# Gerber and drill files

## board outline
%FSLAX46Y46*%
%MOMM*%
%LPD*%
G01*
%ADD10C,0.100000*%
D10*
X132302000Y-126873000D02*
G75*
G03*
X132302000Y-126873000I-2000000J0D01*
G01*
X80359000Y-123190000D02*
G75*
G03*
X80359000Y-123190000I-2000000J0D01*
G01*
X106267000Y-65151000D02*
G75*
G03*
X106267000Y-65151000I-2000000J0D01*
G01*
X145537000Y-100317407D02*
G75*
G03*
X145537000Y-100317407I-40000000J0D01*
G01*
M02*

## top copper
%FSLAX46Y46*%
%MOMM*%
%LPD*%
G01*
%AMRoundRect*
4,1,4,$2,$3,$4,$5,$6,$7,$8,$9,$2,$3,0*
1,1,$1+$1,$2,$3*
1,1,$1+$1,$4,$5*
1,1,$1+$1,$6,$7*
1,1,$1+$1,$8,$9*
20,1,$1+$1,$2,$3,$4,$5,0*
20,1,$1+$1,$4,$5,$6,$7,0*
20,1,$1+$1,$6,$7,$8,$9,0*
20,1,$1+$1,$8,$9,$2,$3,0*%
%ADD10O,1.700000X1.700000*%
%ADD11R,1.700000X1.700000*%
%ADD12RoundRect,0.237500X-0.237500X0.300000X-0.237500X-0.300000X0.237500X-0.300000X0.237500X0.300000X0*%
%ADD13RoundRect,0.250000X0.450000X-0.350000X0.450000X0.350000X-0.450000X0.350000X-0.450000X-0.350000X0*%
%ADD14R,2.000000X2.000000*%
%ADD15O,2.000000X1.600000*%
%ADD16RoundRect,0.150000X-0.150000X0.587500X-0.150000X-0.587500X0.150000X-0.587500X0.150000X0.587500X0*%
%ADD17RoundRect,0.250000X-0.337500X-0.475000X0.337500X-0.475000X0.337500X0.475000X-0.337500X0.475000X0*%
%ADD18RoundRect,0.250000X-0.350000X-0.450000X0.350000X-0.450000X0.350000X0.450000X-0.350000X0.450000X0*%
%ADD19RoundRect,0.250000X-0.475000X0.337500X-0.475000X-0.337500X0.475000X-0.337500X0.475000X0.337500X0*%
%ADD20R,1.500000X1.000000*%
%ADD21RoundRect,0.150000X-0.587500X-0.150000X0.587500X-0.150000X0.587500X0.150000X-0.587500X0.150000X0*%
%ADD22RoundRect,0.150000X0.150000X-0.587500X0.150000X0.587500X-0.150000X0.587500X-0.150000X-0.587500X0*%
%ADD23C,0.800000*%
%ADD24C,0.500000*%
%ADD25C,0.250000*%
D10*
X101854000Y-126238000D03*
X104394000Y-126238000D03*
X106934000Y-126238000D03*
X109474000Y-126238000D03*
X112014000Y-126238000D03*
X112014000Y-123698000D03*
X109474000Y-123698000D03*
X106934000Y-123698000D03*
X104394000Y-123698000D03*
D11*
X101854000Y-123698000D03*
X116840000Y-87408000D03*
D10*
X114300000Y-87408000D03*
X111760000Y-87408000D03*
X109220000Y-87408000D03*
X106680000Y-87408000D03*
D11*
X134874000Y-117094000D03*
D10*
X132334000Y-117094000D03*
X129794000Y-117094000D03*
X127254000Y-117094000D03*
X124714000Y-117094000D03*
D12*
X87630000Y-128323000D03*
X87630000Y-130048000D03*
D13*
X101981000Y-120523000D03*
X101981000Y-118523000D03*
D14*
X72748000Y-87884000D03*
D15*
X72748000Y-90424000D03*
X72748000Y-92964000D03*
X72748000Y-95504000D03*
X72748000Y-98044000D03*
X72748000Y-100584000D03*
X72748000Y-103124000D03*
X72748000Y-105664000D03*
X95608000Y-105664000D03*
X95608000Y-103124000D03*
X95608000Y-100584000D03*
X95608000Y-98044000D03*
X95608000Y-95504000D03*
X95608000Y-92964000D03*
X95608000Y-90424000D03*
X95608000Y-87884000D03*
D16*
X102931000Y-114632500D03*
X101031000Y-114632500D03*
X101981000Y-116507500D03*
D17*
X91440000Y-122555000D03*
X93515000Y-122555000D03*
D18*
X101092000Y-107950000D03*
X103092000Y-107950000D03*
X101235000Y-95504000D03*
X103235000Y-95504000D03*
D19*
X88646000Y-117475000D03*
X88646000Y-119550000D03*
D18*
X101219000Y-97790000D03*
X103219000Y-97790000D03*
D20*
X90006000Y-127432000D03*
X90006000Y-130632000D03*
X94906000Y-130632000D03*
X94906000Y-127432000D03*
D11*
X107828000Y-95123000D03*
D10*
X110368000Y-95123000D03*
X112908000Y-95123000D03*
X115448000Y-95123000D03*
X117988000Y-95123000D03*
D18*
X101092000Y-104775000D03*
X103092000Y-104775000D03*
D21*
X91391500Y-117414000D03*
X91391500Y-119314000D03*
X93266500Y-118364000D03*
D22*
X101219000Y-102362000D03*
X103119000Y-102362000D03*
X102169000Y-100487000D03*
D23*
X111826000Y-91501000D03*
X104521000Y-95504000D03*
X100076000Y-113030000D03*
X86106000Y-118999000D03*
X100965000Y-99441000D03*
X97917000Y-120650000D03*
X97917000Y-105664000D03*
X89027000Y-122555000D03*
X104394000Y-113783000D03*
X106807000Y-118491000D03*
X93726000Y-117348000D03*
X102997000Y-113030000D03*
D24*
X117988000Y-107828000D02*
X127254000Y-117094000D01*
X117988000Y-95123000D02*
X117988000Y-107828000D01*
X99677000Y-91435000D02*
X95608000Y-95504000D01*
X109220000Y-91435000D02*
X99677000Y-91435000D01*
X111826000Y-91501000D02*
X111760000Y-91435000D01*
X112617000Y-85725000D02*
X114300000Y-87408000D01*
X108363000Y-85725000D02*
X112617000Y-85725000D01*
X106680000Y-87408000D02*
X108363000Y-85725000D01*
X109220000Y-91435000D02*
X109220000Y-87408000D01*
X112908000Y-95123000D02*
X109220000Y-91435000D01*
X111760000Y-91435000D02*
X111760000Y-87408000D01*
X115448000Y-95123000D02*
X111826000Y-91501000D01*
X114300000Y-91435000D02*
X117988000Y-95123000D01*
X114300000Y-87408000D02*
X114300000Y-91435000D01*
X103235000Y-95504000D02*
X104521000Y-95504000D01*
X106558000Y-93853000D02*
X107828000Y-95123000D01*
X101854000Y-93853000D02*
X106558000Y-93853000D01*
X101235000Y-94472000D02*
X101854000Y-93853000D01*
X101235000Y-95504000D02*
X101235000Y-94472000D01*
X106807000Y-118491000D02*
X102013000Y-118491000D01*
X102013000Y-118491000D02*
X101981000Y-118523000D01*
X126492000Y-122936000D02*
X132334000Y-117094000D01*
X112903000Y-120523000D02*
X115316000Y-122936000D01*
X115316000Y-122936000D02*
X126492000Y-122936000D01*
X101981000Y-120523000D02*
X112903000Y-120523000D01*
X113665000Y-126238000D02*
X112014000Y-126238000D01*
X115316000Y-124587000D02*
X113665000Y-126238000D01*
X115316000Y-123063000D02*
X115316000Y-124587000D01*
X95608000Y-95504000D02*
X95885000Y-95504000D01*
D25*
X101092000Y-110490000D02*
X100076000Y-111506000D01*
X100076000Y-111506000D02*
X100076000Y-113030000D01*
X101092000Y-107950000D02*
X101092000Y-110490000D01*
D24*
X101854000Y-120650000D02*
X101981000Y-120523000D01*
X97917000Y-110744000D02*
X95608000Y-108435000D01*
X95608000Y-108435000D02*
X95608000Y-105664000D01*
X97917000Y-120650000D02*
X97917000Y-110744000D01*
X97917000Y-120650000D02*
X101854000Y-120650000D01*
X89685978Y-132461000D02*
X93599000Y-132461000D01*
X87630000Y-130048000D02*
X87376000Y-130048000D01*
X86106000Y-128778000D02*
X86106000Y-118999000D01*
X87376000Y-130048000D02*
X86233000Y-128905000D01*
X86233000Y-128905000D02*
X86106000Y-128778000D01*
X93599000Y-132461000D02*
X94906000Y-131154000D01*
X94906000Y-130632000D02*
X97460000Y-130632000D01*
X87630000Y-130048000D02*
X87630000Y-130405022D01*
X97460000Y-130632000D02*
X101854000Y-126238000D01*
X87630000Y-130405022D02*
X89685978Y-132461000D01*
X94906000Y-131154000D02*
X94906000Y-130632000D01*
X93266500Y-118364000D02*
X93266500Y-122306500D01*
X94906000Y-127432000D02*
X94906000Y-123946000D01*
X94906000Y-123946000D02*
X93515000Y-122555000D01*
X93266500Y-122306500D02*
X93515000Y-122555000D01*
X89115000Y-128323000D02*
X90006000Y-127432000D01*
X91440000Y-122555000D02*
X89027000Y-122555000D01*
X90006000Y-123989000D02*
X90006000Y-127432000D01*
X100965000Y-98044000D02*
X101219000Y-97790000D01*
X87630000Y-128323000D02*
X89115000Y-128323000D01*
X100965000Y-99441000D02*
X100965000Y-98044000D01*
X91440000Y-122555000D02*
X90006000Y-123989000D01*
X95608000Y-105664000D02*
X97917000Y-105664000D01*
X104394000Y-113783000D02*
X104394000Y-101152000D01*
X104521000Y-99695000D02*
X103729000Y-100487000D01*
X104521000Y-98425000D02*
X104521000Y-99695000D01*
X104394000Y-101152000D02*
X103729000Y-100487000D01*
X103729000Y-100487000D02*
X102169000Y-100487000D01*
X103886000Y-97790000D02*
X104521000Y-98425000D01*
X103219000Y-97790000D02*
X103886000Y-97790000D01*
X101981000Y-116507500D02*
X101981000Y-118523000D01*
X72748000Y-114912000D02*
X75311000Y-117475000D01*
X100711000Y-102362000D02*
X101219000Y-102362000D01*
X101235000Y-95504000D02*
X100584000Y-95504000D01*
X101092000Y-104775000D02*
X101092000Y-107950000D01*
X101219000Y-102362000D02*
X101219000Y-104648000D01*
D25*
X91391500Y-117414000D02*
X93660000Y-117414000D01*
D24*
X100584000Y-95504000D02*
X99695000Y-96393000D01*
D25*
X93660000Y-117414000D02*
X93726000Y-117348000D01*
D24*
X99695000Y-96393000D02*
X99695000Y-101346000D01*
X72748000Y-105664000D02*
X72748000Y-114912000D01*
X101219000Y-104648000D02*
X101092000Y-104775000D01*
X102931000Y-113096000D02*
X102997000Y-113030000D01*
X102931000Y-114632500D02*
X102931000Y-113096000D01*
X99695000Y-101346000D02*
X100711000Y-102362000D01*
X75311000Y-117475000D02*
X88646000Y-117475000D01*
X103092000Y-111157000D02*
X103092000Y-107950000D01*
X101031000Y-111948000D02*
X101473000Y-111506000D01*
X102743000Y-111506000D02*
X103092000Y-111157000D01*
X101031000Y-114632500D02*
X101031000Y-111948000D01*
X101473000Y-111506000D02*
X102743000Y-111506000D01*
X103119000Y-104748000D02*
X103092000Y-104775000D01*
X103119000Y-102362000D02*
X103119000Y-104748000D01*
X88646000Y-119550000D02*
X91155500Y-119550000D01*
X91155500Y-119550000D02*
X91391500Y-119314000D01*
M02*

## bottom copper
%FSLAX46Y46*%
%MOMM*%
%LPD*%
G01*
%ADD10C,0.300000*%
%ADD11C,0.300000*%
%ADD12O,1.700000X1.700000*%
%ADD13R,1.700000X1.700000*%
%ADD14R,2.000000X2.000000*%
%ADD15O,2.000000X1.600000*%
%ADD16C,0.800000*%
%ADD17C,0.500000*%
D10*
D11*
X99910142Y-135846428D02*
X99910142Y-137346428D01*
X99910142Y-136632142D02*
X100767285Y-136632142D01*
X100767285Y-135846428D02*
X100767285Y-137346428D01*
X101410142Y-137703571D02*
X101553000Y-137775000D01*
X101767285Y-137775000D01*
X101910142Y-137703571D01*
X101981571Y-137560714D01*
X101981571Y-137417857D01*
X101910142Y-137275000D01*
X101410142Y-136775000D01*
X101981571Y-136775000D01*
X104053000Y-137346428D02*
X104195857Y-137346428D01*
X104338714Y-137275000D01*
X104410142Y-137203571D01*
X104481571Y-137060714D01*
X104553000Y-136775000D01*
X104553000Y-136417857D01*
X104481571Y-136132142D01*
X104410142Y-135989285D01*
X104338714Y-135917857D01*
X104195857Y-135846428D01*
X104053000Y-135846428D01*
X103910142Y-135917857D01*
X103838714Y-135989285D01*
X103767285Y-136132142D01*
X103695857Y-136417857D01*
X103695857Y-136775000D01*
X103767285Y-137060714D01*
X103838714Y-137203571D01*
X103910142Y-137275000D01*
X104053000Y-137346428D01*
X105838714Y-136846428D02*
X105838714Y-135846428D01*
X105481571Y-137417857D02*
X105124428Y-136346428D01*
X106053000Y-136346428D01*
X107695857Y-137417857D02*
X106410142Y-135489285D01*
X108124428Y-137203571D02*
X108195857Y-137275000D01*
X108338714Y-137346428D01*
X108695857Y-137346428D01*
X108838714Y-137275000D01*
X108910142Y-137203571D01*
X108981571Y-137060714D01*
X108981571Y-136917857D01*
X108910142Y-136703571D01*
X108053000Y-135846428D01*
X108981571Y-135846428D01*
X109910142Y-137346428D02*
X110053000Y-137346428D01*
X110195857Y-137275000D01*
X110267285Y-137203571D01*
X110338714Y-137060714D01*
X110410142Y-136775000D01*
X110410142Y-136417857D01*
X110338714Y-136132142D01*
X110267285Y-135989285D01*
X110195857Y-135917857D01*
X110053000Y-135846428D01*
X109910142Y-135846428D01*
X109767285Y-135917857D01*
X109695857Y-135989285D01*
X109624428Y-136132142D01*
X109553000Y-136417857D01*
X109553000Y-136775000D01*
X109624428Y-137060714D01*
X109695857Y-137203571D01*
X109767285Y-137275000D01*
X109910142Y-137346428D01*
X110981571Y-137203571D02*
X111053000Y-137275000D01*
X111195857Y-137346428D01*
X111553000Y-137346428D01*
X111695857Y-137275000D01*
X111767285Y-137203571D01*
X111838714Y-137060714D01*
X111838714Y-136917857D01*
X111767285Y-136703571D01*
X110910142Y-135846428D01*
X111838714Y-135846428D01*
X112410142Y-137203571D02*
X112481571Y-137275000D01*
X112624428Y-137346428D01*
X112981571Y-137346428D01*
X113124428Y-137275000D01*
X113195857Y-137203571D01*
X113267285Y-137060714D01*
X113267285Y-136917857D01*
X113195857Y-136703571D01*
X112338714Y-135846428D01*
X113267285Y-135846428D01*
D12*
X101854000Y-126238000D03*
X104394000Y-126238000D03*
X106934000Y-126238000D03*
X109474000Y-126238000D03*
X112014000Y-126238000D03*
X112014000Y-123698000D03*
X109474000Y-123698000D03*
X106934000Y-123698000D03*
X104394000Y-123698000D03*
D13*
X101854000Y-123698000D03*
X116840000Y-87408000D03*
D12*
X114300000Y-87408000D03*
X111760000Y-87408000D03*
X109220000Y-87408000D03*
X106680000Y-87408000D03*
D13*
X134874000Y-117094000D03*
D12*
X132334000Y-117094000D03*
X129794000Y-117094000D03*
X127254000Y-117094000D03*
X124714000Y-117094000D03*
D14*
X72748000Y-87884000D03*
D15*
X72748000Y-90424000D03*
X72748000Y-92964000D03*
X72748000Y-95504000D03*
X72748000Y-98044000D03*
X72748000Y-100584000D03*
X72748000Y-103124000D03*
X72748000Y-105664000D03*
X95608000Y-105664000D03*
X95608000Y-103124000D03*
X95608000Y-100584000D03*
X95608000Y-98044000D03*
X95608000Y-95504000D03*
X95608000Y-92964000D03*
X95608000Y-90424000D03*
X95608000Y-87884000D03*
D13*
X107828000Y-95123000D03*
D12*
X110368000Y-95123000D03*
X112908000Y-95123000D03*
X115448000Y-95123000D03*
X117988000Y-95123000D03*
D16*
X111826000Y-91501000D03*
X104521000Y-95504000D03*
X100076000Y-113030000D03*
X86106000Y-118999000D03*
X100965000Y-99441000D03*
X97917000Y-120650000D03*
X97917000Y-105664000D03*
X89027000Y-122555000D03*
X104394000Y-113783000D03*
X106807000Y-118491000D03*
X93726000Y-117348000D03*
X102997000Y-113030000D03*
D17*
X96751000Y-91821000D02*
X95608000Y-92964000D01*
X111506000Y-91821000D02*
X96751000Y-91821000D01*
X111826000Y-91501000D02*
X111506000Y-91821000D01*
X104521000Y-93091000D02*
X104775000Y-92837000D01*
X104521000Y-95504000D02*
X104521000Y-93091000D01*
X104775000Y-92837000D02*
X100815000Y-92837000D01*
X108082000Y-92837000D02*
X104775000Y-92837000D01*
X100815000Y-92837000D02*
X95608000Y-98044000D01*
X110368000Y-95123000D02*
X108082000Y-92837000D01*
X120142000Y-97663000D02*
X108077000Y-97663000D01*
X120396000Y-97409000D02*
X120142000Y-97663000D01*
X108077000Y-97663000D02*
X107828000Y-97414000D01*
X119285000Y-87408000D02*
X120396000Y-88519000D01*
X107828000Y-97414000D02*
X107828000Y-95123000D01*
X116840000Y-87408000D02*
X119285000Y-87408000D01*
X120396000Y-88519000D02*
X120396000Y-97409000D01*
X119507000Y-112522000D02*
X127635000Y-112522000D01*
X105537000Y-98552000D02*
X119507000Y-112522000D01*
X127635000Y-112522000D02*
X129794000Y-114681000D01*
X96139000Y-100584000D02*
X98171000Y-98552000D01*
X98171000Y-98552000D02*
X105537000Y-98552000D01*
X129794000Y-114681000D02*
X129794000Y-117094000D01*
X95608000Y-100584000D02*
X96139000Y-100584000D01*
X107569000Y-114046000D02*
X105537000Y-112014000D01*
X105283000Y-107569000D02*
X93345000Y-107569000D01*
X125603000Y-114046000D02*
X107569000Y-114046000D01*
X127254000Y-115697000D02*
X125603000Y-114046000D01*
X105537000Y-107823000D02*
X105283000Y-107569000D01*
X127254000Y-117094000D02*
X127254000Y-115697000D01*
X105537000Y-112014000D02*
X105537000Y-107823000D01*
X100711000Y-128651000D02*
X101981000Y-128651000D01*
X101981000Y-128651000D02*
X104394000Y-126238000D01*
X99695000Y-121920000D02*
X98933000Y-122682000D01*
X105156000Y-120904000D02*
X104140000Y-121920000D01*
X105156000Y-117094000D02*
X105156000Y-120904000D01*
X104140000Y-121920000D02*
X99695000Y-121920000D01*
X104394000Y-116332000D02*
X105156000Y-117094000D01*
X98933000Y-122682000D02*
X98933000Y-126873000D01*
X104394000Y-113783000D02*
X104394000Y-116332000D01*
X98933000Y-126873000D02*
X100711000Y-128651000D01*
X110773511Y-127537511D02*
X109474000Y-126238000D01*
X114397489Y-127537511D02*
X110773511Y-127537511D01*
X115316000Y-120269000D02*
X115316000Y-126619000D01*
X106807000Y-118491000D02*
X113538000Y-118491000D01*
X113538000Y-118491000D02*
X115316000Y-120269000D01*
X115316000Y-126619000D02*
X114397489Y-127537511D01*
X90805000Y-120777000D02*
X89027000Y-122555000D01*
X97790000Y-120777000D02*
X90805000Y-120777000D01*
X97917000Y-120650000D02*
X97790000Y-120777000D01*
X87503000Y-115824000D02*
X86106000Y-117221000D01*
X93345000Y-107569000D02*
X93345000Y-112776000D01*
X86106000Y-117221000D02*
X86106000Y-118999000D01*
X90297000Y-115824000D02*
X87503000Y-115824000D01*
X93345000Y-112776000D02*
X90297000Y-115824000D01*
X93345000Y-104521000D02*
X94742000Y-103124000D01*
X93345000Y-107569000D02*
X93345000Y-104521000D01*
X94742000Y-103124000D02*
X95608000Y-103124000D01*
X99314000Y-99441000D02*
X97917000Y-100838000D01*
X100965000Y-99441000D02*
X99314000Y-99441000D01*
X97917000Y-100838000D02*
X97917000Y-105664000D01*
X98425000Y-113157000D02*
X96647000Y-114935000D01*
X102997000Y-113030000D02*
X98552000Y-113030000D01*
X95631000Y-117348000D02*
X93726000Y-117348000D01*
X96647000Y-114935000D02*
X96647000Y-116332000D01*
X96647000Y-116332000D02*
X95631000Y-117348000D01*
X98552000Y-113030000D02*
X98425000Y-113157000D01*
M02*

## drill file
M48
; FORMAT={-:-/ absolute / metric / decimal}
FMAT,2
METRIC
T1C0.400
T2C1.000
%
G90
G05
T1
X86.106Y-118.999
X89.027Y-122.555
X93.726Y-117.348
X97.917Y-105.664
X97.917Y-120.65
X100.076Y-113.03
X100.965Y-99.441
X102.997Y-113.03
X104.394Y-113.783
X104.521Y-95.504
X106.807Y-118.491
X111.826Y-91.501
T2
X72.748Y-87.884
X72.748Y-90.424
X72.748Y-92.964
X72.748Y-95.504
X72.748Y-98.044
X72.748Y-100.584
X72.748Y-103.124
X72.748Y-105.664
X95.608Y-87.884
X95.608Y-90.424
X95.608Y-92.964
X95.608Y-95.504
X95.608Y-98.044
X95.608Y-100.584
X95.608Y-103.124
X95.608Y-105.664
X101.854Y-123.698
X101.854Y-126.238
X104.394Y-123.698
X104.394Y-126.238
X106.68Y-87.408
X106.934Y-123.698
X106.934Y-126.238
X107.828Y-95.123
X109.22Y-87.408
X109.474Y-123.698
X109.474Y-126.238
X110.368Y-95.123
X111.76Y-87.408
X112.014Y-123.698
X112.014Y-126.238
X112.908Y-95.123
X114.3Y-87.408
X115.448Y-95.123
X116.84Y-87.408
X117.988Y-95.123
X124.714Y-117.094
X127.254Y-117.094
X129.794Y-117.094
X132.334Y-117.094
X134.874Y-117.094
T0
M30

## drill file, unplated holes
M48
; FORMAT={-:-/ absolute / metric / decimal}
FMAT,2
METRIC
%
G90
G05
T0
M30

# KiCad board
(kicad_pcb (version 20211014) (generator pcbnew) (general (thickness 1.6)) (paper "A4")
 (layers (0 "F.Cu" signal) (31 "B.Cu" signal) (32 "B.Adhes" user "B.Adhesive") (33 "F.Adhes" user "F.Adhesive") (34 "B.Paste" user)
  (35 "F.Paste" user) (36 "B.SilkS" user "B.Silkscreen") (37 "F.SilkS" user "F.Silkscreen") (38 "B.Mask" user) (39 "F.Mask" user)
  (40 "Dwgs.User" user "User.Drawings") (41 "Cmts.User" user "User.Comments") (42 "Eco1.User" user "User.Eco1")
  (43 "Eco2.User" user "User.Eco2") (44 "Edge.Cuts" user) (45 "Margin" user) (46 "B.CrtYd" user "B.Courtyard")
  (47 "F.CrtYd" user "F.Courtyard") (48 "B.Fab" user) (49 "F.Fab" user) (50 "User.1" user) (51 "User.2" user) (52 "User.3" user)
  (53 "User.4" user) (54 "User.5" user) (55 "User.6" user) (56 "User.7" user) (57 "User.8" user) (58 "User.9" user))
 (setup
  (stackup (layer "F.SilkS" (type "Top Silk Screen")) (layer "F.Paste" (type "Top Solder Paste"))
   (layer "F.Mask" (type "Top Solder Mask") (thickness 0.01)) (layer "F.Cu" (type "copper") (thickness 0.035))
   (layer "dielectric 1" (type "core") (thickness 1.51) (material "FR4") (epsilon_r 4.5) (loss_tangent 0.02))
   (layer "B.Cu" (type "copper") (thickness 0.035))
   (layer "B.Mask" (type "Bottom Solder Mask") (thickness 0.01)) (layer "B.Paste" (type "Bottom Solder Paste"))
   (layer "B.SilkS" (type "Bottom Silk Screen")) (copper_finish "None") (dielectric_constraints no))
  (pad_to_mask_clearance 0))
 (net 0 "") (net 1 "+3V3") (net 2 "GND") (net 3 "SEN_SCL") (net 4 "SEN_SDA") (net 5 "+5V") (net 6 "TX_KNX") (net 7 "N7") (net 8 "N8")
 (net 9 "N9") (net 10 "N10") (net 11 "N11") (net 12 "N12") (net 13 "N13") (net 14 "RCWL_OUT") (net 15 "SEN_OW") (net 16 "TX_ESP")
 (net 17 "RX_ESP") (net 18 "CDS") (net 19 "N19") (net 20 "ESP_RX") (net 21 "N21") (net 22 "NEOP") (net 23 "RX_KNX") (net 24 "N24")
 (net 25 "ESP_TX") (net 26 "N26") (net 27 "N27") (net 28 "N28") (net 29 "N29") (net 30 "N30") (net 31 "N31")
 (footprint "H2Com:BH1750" (layer "F.Cu") (at 116.84 100.108 -90)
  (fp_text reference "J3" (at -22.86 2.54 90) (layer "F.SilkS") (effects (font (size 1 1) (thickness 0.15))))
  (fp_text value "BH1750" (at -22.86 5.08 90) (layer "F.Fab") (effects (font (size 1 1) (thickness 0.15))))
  (pad "1" thru_hole rect (at -12.7 0 270) (size 1.7 1.7) (drill 1) (layers *.Cu *.Mask) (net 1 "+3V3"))
  (pad "2" thru_hole oval (at -12.7 2.54 270) (size 1.7 1.7) (drill 1) (layers *.Cu *.Mask) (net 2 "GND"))
  (pad "3" thru_hole oval (at -12.7 5.08 270) (size 1.7 1.7) (drill 1) (layers *.Cu *.Mask) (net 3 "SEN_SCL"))
  (pad "4" thru_hole oval (at -12.7 7.62 270) (size 1.7 1.7) (drill 1) (layers *.Cu *.Mask) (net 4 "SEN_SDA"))
  (pad "5" thru_hole oval (at -12.7 10.16 270) (size 1.7 1.7) (drill 1) (layers *.Cu *.Mask) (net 2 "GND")))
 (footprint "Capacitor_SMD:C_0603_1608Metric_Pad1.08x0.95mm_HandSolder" (layer "F.Cu") (at 87.63 129.1855 -90)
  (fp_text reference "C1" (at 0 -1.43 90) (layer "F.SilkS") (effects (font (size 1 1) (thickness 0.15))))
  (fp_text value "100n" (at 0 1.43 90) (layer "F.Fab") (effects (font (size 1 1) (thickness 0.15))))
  (pad "1" smd roundrect locked (at -0.8625 0 270) (size 1.075 0.95) (layers "F.Cu" "F.Paste" "F.Mask") (roundrect_rratio 0.25)
   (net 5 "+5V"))
  (pad "2" smd roundrect locked (at 0.8625 0 270) (size 1.075 0.95) (layers "F.Cu" "F.Paste" "F.Mask") (roundrect_rratio 0.25) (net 2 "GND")))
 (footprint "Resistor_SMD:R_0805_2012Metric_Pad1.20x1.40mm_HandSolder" (layer "F.Cu") (at 101.981 119.523 90)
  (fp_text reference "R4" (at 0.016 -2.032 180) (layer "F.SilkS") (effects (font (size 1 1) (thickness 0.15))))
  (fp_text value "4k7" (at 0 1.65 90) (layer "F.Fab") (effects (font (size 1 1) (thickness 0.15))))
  (pad "1" smd roundrect locked (at -1 0 90) (size 1.2 1.4) (layers "F.Cu" "F.Paste" "F.Mask") (roundrect_rratio 0.2083333333) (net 5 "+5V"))
  (pad "2" smd roundrect locked (at 1 0 90) (size 1.2 1.4) (layers "F.Cu" "F.Paste" "F.Mask") (roundrect_rratio 0.2083333333)
   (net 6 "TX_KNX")))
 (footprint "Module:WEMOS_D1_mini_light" (layer "F.Cu") (at 72.748 87.884)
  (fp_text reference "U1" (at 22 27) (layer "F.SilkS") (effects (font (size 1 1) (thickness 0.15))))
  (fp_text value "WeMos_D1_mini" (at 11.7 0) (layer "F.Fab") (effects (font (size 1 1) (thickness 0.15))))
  (pad "1" thru_hole rect locked (at 0 0) (size 2 2) (drill 1) (layers *.Cu *.Mask) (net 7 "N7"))
  (pad "2" thru_hole oval locked (at 0 2.54) (size 2 1.6) (drill 1) (layers *.Cu *.Mask) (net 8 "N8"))
  (pad "3" thru_hole oval locked (at 0 5.08) (size 2 1.6) (drill 1) (layers *.Cu *.Mask) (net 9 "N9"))
  (pad "4" thru_hole oval locked (at 0 7.62) (size 2 1.6) (drill 1) (layers *.Cu *.Mask) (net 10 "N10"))
  (pad "5" thru_hole oval locked (at 0 10.16) (size 2 1.6) (drill 1) (layers *.Cu *.Mask) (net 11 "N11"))
  (pad "6" thru_hole oval locked (at 0 12.7) (size 2 1.6) (drill 1) (layers *.Cu *.Mask) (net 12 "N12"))
  (pad "7" thru_hole oval locked (at 0 15.24) (size 2 1.6) (drill 1) (layers *.Cu *.Mask) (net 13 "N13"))
  (pad "8" thru_hole oval locked (at 0 17.78) (size 2 1.6) (drill 1) (layers *.Cu *.Mask) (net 1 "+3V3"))
  (pad "9" thru_hole oval locked (at 22.86 17.78) (size 2 1.6) (drill 1) (layers *.Cu *.Mask) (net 5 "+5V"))
  (pad "10" thru_hole oval locked (at 22.86 15.24) (size 2 1.6) (drill 1) (layers *.Cu *.Mask) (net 2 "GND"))
  (pad "11" thru_hole oval locked (at 22.86 12.7) (size 2 1.6) (drill 1) (layers *.Cu *.Mask) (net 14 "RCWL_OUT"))
  (pad "12" thru_hole oval locked (at 22.86 10.16) (size 2 1.6) (drill 1) (layers *.Cu *.Mask) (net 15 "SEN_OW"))
  (pad "13" thru_hole oval locked (at 22.86 7.62) (size 2 1.6) (drill 1) (layers *.Cu *.Mask) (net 4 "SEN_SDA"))
  (pad "14" thru_hole oval locked (at 22.86 5.08) (size 2 1.6) (drill 1) (layers *.Cu *.Mask) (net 3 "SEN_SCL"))
  (pad "15" thru_hole oval locked (at 22.86 2.54) (size 2 1.6) (drill 1) (layers *.Cu *.Mask) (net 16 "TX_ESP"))
  (pad "16" thru_hole oval locked (at 22.86 0) (size 2 1.6) (drill 1) (layers *.Cu *.Mask) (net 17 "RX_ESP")))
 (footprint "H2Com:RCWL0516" (layer "F.Cu") (at 123.444 101.854 -90)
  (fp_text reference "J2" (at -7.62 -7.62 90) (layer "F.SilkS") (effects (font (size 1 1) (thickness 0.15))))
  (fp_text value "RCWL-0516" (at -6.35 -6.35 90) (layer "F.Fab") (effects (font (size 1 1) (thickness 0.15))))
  (pad "1" thru_hole rect (at 15.24 -11.43 270) (size 1.7 1.7) (drill 1) (layers *.Cu *.Mask) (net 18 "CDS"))
  (pad "2" thru_hole oval (at 15.24 -8.89 270) (size 1.7 1.7) (drill 1) (layers *.Cu *.Mask) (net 5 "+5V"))
  (pad "3" thru_hole oval (at 15.24 -6.35 270) (size 1.7 1.7) (drill 1) (layers *.Cu *.Mask) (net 14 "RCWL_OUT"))
  (pad "4" thru_hole oval (at 15.24 -3.81 270) (size 1.7 1.7) (drill 1) (layers *.Cu *.Mask) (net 2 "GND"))
  (pad "5" thru_hole oval (at 15.24 -1.27 270) (size 1.7 1.7) (drill 1) (layers *.Cu *.Mask) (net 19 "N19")))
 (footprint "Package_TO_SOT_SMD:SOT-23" (layer "F.Cu") (at 101.981 115.57 -90)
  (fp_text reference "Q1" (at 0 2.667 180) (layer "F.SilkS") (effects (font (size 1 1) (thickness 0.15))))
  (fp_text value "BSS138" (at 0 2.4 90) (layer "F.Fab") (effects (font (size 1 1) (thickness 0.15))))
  (pad "1" smd roundrect locked (at -0.9375 -0.95 270) (size 1.475 0.6) (layers "F.Cu" "F.Paste" "F.Mask") (roundrect_rratio 0.25)
   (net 1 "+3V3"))
  (pad "2" smd roundrect locked (at -0.9375 0.95 270) (size 1.475 0.6) (layers "F.Cu" "F.Paste" "F.Mask") (roundrect_rratio 0.25)
   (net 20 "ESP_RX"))
  (pad "3" smd roundrect locked (at 0.9375 0 270) (size 1.475 0.6) (layers "F.Cu" "F.Paste" "F.Mask") (roundrect_rratio 0.25)
   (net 6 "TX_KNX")))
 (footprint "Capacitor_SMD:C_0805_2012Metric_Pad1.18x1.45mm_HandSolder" (layer "F.Cu") (at 92.4775 122.555)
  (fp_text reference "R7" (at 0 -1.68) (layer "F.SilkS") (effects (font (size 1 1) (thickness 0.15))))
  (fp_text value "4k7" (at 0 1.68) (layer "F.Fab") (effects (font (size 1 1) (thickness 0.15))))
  (pad "1" smd roundrect locked (at -1.0375 0) (size 1.175 1.45) (layers "F.Cu" "F.Paste" "F.Mask") (roundrect_rratio 0.2127659574)
   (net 5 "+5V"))
  (pad "2" smd roundrect locked (at 1.0375 0) (size 1.175 1.45) (layers "F.Cu" "F.Paste" "F.Mask") (roundrect_rratio 0.2127659574)
   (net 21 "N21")))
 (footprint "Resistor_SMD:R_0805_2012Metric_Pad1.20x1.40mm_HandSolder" (layer "F.Cu") (at 102.092 107.95)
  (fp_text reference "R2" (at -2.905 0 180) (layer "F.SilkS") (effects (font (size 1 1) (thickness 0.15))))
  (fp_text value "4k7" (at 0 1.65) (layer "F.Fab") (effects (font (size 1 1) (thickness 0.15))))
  (pad "1" smd roundrect locked (at -1 0) (size 1.2 1.4) (layers "F.Cu" "F.Paste" "F.Mask") (roundrect_rratio 0.2083333333) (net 1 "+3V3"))
  (pad "2" smd roundrect locked (at 1 0) (size 1.2 1.4) (layers "F.Cu" "F.Paste" "F.Mask") (roundrect_rratio 0.2083333333) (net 20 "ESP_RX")))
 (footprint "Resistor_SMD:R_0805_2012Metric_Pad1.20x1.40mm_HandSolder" (layer "F.Cu") (at 102.235 95.504)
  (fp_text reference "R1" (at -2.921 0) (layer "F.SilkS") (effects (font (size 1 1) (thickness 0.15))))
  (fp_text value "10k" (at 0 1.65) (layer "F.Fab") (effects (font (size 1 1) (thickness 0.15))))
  (pad "1" smd roundrect locked (at -1 0) (size 1.2 1.4) (layers "F.Cu" "F.Paste" "F.Mask") (roundrect_rratio 0.2083333333) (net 1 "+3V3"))
  (pad "2" smd roundrect locked (at 1 0) (size 1.2 1.4) (layers "F.Cu" "F.Paste" "F.Mask") (roundrect_rratio 0.2083333333) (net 15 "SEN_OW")))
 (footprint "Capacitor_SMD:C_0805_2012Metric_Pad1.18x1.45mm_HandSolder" (layer "F.Cu") (at 88.646 118.5125 -90)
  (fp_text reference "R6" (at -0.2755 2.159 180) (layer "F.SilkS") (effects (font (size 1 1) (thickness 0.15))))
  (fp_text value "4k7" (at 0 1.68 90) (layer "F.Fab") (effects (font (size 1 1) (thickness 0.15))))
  (pad "1" smd roundrect locked (at -1.0375 0 270) (size 1.175 1.45) (layers "F.Cu" "F.Paste" "F.Mask") (roundrect_rratio 0.2127659574)
   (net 1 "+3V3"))
  (pad "2" smd roundrect locked (at 1.0375 0 270) (size 1.175 1.45) (layers "F.Cu" "F.Paste" "F.Mask") (roundrect_rratio 0.2127659574)
   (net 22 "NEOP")))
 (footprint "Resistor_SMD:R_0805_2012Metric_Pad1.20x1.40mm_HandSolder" (layer "F.Cu") (at 102.219 97.79)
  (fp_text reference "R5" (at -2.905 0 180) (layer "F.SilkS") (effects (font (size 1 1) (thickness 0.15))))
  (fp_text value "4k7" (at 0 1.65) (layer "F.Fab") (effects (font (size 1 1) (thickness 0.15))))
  (pad "1" smd roundrect locked (at -1 0) (size 1.2 1.4) (layers "F.Cu" "F.Paste" "F.Mask") (roundrect_rratio 0.2083333333) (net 5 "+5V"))
  (pad "2" smd roundrect locked (at 1 0) (size 1.2 1.4) (layers "F.Cu" "F.Paste" "F.Mask") (roundrect_rratio 0.2083333333) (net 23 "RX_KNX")))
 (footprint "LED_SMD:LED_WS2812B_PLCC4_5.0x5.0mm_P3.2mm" (layer "F.Cu") (at 92.456 129.032)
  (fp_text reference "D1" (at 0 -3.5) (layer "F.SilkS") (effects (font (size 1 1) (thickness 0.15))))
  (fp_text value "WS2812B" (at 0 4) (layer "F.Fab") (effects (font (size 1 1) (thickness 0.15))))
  (pad "1" smd rect locked (at -2.45 -1.6) (size 1.5 1) (layers "F.Cu" "F.Paste" "F.Mask") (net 5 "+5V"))
  (pad "2" smd rect locked (at -2.45 1.6) (size 1.5 1) (layers "F.Cu" "F.Paste" "F.Mask") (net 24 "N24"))
  (pad "3" smd rect locked (at 2.45 1.6) (size 1.5 1) (layers "F.Cu" "F.Paste" "F.Mask") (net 2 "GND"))
  (pad "4" smd rect locked (at 2.45 -1.6) (size 1.5 1) (layers "F.Cu" "F.Paste" "F.Mask") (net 21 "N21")))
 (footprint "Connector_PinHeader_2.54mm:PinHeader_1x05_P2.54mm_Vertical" (layer "F.Cu") (at 107.828 95.123 90)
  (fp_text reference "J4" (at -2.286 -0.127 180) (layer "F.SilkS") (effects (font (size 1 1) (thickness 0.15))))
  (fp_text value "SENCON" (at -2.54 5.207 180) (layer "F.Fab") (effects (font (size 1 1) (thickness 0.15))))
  (pad "1" thru_hole rect locked (at 0 0 90) (size 1.7 1.7) (drill 1) (layers *.Cu *.Mask) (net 1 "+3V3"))
  (pad "2" thru_hole oval locked (at 0 2.54 90) (size 1.7 1.7) (drill 1) (layers *.Cu *.Mask) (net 15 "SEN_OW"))
  (pad "3" thru_hole oval locked (at 0 5.08 90) (size 1.7 1.7) (drill 1) (layers *.Cu *.Mask) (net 4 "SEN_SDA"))
  (pad "4" thru_hole oval locked (at 0 7.62 90) (size 1.7 1.7) (drill 1) (layers *.Cu *.Mask) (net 3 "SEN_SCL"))
  (pad "5" thru_hole oval locked (at 0 10.16 90) (size 1.7 1.7) (drill 1) (layers *.Cu *.Mask) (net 2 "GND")))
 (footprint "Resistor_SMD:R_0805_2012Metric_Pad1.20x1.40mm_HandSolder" (layer "F.Cu") (at 102.092 104.775)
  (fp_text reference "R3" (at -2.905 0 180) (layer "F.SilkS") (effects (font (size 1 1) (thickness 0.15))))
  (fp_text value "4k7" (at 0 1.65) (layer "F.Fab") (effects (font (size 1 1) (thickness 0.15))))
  (pad "1" smd roundrect locked (at -1 0) (size 1.2 1.4) (layers "F.Cu" "F.Paste" "F.Mask") (roundrect_rratio 0.2083333333) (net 1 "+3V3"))
  (pad "2" smd roundrect locked (at 1 0) (size 1.2 1.4) (layers "F.Cu" "F.Paste" "F.Mask") (roundrect_rratio 0.2083333333) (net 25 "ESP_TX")))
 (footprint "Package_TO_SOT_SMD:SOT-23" (layer "F.Cu") (at 92.329 118.364)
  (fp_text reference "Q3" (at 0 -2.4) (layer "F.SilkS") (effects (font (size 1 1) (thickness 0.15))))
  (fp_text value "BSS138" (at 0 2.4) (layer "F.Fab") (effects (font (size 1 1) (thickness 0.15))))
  (pad "1" smd roundrect locked (at -0.9375 -0.95) (size 1.475 0.6) (layers "F.Cu" "F.Paste" "F.Mask") (roundrect_rratio 0.25)
   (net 1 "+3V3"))
  (pad "2" smd roundrect locked (at -0.9375 0.95) (size 1.475 0.6) (layers "F.Cu" "F.Paste" "F.Mask") (roundrect_rratio 0.25)
   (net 22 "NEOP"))
  (pad "3" smd roundrect locked (at 0.9375 0) (size 1.475 0.6) (layers "F.Cu" "F.Paste" "F.Mask") (roundrect_rratio 0.25) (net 21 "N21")))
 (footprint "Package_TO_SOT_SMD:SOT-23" (layer "F.Cu") (at 102.169 101.4245 90)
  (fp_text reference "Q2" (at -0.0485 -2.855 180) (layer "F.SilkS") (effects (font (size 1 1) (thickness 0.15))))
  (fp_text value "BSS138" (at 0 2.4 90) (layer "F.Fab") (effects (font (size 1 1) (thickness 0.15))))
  (pad "1" smd roundrect locked (at -0.9375 -0.95 90) (size 1.475 0.6) (layers "F.Cu" "F.Paste" "F.Mask") (roundrect_rratio 0.25)
   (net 1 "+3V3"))
  (pad "2" smd roundrect locked (at -0.9375 0.95 90) (size 1.475 0.6) (layers "F.Cu" "F.Paste" "F.Mask") (roundrect_rratio 0.25)
   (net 25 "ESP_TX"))
  (pad "3" smd roundrect locked (at 0.9375 0 90) (size 1.475 0.6) (layers "F.Cu" "F.Paste" "F.Mask") (roundrect_rratio 0.25)
   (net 23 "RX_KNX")))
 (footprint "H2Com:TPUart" (layer "B.Cu") (at 101.854 126.238 -90)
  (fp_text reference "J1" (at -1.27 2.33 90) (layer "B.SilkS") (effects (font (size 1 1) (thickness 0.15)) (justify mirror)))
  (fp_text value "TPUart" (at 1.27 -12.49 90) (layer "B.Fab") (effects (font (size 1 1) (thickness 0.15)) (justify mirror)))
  (pad "1" thru_hole oval (at 0 0 270) (size 1.7 1.7) (drill 1) (layers *.Cu *.Mask) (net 2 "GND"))
  (pad "2" thru_hole oval (at 0 -2.54 270) (size 1.7 1.7) (drill 1) (layers *.Cu *.Mask) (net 23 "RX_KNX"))
  (pad "3" thru_hole oval (at 0 -5.08 270) (size 1.7 1.7) (drill 1) (layers *.Cu *.Mask) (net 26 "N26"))
  (pad "4" thru_hole oval (at 0 -7.62 270) (size 1.7 1.7) (drill 1) (layers *.Cu *.Mask) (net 6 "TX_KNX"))
  (pad "5" thru_hole oval (at 0 -10.16 270) (size 1.7 1.7) (drill 1) (layers *.Cu *.Mask) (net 5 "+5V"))
  (pad "6" thru_hole oval (at -2.54 -10.16 270) (size 1.7 1.7) (drill 1) (layers *.Cu *.Mask) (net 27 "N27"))
  (pad "7" thru_hole oval (at -2.54 -7.62 270) (size 1.7 1.7) (drill 1) (layers *.Cu *.Mask) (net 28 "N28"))
  (pad "8" thru_hole oval (at -2.54 -5.08 270) (size 1.7 1.7) (drill 1) (layers *.Cu *.Mask) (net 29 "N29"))
  (pad "9" thru_hole oval (at -2.54 -2.54 270) (size 1.7 1.7) (drill 1) (layers *.Cu *.Mask) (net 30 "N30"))
  (pad "10" thru_hole rect (at -2.54 0 270) (size 1.7 1.7) (drill 1) (layers *.Cu *.Mask) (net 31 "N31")))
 (gr_circle (center 78.359 123.19) (end 80.359 123.19) (layer "Edge.Cuts") (width 0.1) (fill none))
 (gr_circle (center 104.267 65.151) (end 106.267 65.151) (layer "Edge.Cuts") (width 0.1) (fill none))
 (gr_circle (center 130.302 126.873) (end 132.302 126.873) (layer "Edge.Cuts") (width 0.1) (fill none))
 (gr_circle (center 105.537 100.317407) (end 145.537 100.317407) (layer "Edge.Cuts") (width 0.1) (fill none))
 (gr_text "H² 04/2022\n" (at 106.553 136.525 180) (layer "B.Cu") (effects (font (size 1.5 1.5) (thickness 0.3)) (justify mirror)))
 (segment (start 89.685978 132.461) (end 93.599 132.461) (width 0.5) (layer "F.Cu") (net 2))
 (segment (start 117.988 95.123) (end 117.988 107.828) (width 0.5) (layer "F.Cu") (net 2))
 (segment (start 87.63 130.048) (end 87.376 130.048) (width 0.5) (layer "F.Cu") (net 2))
 (segment (start 112.617 85.725) (end 114.3 87.408) (width 0.5) (layer "F.Cu") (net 2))
 (segment (start 86.106 128.778) (end 86.106 118.999) (width 0.5) (layer "F.Cu") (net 2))
 (segment (start 117.988 107.828) (end 127.254 117.094) (width 0.5) (layer "F.Cu") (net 2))
 (segment (start 87.376 130.048) (end 86.233 128.905) (width 0.5) (layer "F.Cu") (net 2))
 (segment (start 86.233 128.905) (end 86.106 128.778) (width 0.5) (layer "F.Cu") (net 2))
 (segment (start 106.68 87.408) (end 108.363 85.725) (width 0.5) (layer "F.Cu") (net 2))
 (segment (start 93.599 132.461) (end 94.906 131.154) (width 0.5) (layer "F.Cu") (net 2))
 (segment (start 94.906 130.632) (end 97.46 130.632) (width 0.5) (layer "F.Cu") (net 2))
 (segment (start 114.3 87.408) (end 114.3 91.435) (width 0.5) (layer "F.Cu") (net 2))
 (segment (start 87.63 130.048) (end 87.63 130.405022) (width 0.5) (layer "F.Cu") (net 2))
 (segment (start 97.46 130.632) (end 101.854 126.238) (width 0.5) (layer "F.Cu") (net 2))
 (segment (start 108.363 85.725) (end 112.617 85.725) (width 0.5) (layer "F.Cu") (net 2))
 (segment (start 114.3 91.435) (end 117.988 95.123) (width 0.5) (layer "F.Cu") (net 2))
 (segment (start 87.63 130.405022) (end 89.685978 132.461) (width 0.5) (layer "F.Cu") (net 2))
 (segment (start 94.906 131.154) (end 94.906 130.632) (width 0.5) (layer "F.Cu") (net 2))
 (via (at 86.106 118.999) (size 0.8) (drill 0.4) (layers "F.Cu" "B.Cu") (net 2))
 (segment (start 87.503 115.824) (end 86.106 117.221) (width 0.5) (layer "B.Cu") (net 2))
 (segment (start 107.569 114.046) (end 105.537 112.014) (width 0.5) (layer "B.Cu") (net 2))
 (segment (start 93.345 107.569) (end 93.345 112.776) (width 0.5) (layer "B.Cu") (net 2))
 (segment (start 86.106 117.221) (end 86.106 118.999) (width 0.5) (layer "B.Cu") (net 2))
 (segment (start 90.297 115.824) (end 87.503 115.824) (width 0.5) (layer "B.Cu") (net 2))
 (segment (start 93.345 112.776) (end 90.297 115.824) (width 0.5) (layer "B.Cu") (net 2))
 (segment (start 93.345 104.521) (end 94.742 103.124) (width 0.5) (layer "B.Cu") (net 2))
 (segment (start 127.254 117.094) (end 127.254 115.697) (width 0.5) (layer "B.Cu") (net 2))
 (segment (start 93.345 107.569) (end 93.345 104.521) (width 0.5) (layer "B.Cu") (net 2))
 (segment (start 94.742 103.124) (end 95.608 103.124) (width 0.5) (layer "B.Cu") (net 2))
 (segment (start 127.254 115.697) (end 125.603 114.046) (width 0.5) (layer "B.Cu") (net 2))
 (segment (start 105.537 107.823) (end 105.283 107.569) (width 0.5) (layer "B.Cu") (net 2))
 (segment (start 125.603 114.046) (end 107.569 114.046) (width 0.5) (layer "B.Cu") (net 2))
 (segment (start 105.537 112.014) (end 105.537 107.823) (width 0.5) (layer "B.Cu") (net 2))
 (segment (start 105.283 107.569) (end 93.345 107.569) (width 0.5) (layer "B.Cu") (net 2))
 (segment (start 93.2665 118.364) (end 93.2665 122.3065) (width 0.5) (layer "F.Cu") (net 21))
 (segment (start 94.906 127.432) (end 94.906 123.946) (width 0.5) (layer "F.Cu") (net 21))
 (segment (start 94.906 123.946) (end 93.515 122.555) (width 0.5) (layer "F.Cu") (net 21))
 (segment (start 93.2665 122.3065) (end 93.515 122.555) (width 0.5) (layer "F.Cu") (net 21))
 (segment (start 126.492 122.936) (end 132.334 117.094) (width 0.5) (layer "F.Cu") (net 5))
 (segment (start 97.917 110.744) (end 95.608 108.435) (width 0.5) (layer "F.Cu") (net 5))
 (segment (start 115.316 124.587) (end 113.665 126.238) (width 0.5) (layer "F.Cu") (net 5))
 (segment (start 97.917 120.65) (end 101.854 120.65) (width 0.5) (layer "F.Cu") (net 5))
 (segment (start 89.115 128.323) (end 90.006 127.432) (width 0.5) (layer "F.Cu") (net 5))
 (segment (start 91.44 122.555) (end 89.027 122.555) (width 0.5) (layer "F.Cu") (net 5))
 (segment (start 90.006 123.989) (end 90.006 127.432) (width 0.5) (layer "F.Cu") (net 5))
 (segment (start 100.965 98.044) (end 101.219 97.79) (width 0.5) (layer "F.Cu") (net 5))
 (segment (start 101.854 120.65) (end 101.981 120.523) (width 0.5) (layer "F.Cu") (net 5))
 (segment (start 87.63 128.323) (end 89.115 128.323) (width 0.5) (layer "F.Cu") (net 5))
 (segment (start 95.608 108.435) (end 95.608 105.664) (width 0.5) (layer "F.Cu") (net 5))
 (segment (start 113.665 126.238) (end 112.014 126.238) (width 0.5) (layer "F.Cu") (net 5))
 (segment (start 100.965 99.441) (end 100.965 98.044) (width 0.5) (layer "F.Cu") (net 5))
 (segment (start 97.917 120.65) (end 97.917 110.744) (width 0.5) (layer "F.Cu") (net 5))
 (segment (start 91.44 122.555) (end 90.006 123.989) (width 0.5) (layer "F.Cu") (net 5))
 (segment (start 112.903 120.523) (end 115.316 122.936) (width 0.5) (layer "F.Cu") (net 5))
 (segment (start 115.316 123.063) (end 115.316 124.587) (width 0.5) (layer "F.Cu") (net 5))
 (segment (start 95.608 105.664) (end 97.917 105.664) (width 0.5) (layer "F.Cu") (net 5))
 (segment (start 101.981 120.523) (end 112.903 120.523) (width 0.5) (layer "F.Cu") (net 5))
 (segment (start 115.316 122.936) (end 126.492 122.936) (width 0.5) (layer "F.Cu") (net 5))
 (via (at 100.965 99.441) (size 0.8) (drill 0.4) (layers "F.Cu" "B.Cu") (free) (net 5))
 (via (at 97.917 120.65) (size 0.8) (drill 0.4) (layers "F.Cu" "B.Cu") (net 5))
 (via (at 97.917 105.664) (size 0.8) (drill 0.4) (layers "F.Cu" "B.Cu") (free) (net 5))
 (via (at 89.027 122.555) (size 0.8) (drill 0.4) (layers "F.Cu" "B.Cu") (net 5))
 (segment (start 99.314 99.441) (end 97.917 100.838) (width 0.5) (layer "B.Cu") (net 5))
 (segment (start 90.805 120.777) (end 89.027 122.555) (width 0.5) (layer "B.Cu") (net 5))
 (segment (start 100.965 99.441) (end 99.314 99.441) (width 0.5) (layer "B.Cu") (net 5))
 (segment (start 97.917 120.65) (end 97.79 120.777) (width 0.5) (layer "B.Cu") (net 5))
 (segment (start 97.79 120.777) (end 90.805 120.777) (width 0.5) (layer "B.Cu") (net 5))
 (segment (start 97.917 100.838) (end 97.917 105.664) (width 0.5) (layer "B.Cu") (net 5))
 (segment (start 127.635 112.522) (end 129.794 114.681) (width 0.5) (layer "B.Cu") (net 14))
 (segment (start 105.537 98.552) (end 119.507 112.522) (width 0.5) (layer "B.Cu") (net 14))
 (segment (start 95.608 100.584) (end 96.139 100.584) (width 0.5) (layer "B.Cu") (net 14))
 (segment (start 129.794 114.681) (end 129.794 117.094) (width 0.5) (layer "B.Cu") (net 14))
 (segment (start 119.507 112.522) (end 127.635 112.522) (width 0.5) (layer "B.Cu") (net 14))
 (segment (start 98.171 98.552) (end 105.537 98.552) (width 0.5) (layer "B.Cu") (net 14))
 (segment (start 96.139 100.584) (end 98.171 98.552) (width 0.5) (layer "B.Cu") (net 14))
 (segment (start 104.394 113.783) (end 104.394 101.152) (width 0.5) (layer "F.Cu") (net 23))
 (segment (start 104.521 99.695) (end 103.729 100.487) (width 0.5) (layer "F.Cu") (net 23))
 (segment (start 104.521 98.425) (end 104.521 99.695) (width 0.5) (layer "F.Cu") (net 23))
 (segment (start 104.394 101.152) (end 103.729 100.487) (width 0.5) (layer "F.Cu") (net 23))
 (segment (start 103.729 100.487) (end 102.169 100.487) (width 0.5) (layer "F.Cu") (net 23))
 (segment (start 103.886 97.79) (end 104.521 98.425) (width 0.5) (layer "F.Cu") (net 23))
 (segment (start 103.219 97.79) (end 103.886 97.79) (width 0.5) (layer "F.Cu") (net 23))
 (via (at 104.394 113.783) (size 0.8) (drill 0.4) (layers "F.Cu" "B.Cu") (free) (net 23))
 (segment (start 104.394 116.332) (end 105.156 117.094) (width 0.5) (layer "B.Cu") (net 23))
 (segment (start 104.14 121.92) (end 99.695 121.92) (width 0.5) (layer "B.Cu") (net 23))
 (segment (start 105.156 120.904) (end 104.14 121.92) (width 0.5) (layer "B.Cu") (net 23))
 (segment (start 98.933 126.873) (end 100.711 128.651) (width 0.5) (layer "B.Cu") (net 23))
 (segment (start 99.695 121.92) (end 98.933 122.682) (width 0.5) (layer "B.Cu") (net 23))
 (segment (start 98.933 122.682) (end 98.933 126.873) (width 0.5) (layer "B.Cu") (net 23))
 (segment (start 105.156 117.094) (end 105.156 120.904) (width 0.5) (layer "B.Cu") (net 23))
 (segment (start 101.981 128.651) (end 104.394 126.238) (width 0.5) (layer "B.Cu") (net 23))
 (segment (start 100.711 128.651) (end 101.981 128.651) (width 0.5) (layer "B.Cu") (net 23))
 (segment (start 104.394 113.783) (end 104.394 116.332) (width 0.5) (layer "B.Cu") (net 23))
 (segment (start 102.013 118.491) (end 101.981 118.523) (width 0.5) (layer "F.Cu") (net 6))
 (segment (start 106.807 118.491) (end 102.013 118.491) (width 0.5) (layer "F.Cu") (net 6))
 (segment (start 101.981 116.5075) (end 101.981 118.523) (width 0.5) (layer "F.Cu") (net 6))
 (via (at 106.807 118.491) (size 0.8) (drill 0.4) (layers "F.Cu" "B.Cu") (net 6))
 (segment (start 115.316 120.269) (end 115.316 126.619) (width 0.5) (layer "B.Cu") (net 6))
 (segment (start 113.538 118.491) (end 115.316 120.269) (width 0.5) (layer "B.Cu") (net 6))
 (segment (start 115.316 126.619) (end 114.397489 127.537511) (width 0.5) (layer "B.Cu") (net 6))
 (segment (start 106.807 118.491) (end 113.538 118.491) (width 0.5) (layer "B.Cu") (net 6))
 (segment (start 110.773511 127.537511) (end 109.474 126.238) (width 0.5) (layer "B.Cu") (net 6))
 (segment (start 114.397489 127.537511) (end 110.773511 127.537511) (width 0.5) (layer "B.Cu") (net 6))
 (segment (start 72.748 114.912) (end 75.311 117.475) (width 0.5) (layer "F.Cu") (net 1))
 (segment (start 100.711 102.362) (end 101.219 102.362) (width 0.5) (layer "F.Cu") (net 1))
 (segment (start 106.558 93.853) (end 107.828 95.123) (width 0.5) (layer "F.Cu") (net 1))
 (segment (start 101.235 95.504) (end 100.584 95.504) (width 0.5) (layer "F.Cu") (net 1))
 (segment (start 101.092 104.775) (end 101.092 107.95) (width 0.5) (layer "F.Cu") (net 1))
 (segment (start 101.092 107.95) (end 101.092 110.49) (width 0.25) (layer "F.Cu") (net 1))
 (segment (start 101.235 94.472) (end 101.854 93.853) (width 0.5) (layer "F.Cu") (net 1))
 (segment (start 101.219 102.362) (end 101.219 104.648) (width 0.5) (layer "F.Cu") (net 1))
 (segment (start 91.3915 117.414) (end 93.66 117.414) (width 0.25) (layer "F.Cu") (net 1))
 (segment (start 101.092 110.49) (end 100.076 111.506) (width 0.25) (layer "F.Cu") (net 1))
 (segment (start 101.235 95.504) (end 101.235 94.472) (width 0.5) (layer "F.Cu") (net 1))
 (segment (start 100.584 95.504) (end 99.695 96.393) (width 0.5) (layer "F.Cu") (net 1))
 (segment (start 93.66 117.414) (end 93.726 117.348) (width 0.25) (layer "F.Cu") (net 1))
 (segment (start 99.695 96.393) (end 99.695 101.346) (width 0.5) (layer "F.Cu") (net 1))
 (segment (start 72.748 105.664) (end 72.748 114.912) (width 0.5) (layer "F.Cu") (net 1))
 (segment (start 101.219 104.648) (end 101.092 104.775) (width 0.5) (layer "F.Cu") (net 1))
 (segment (start 102.931 113.096) (end 102.997 113.03) (width 0.5) (layer "F.Cu") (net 1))
 (segment (start 102.931 114.6325) (end 102.931 113.096) (width 0.5) (layer "F.Cu") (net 1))
 (segment (start 100.076 111.506) (end 100.076 113.03) (width 0.25) (layer "F.Cu") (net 1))
 (segment (start 101.854 93.853) (end 106.558 93.853) (width 0.5) (layer "F.Cu") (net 1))
 (segment (start 99.695 101.346) (end 100.711 102.362) (width 0.5) (layer "F.Cu") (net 1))
 (segment (start 75.311 117.475) (end 88.646 117.475) (width 0.5) (layer "F.Cu") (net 1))
 (via (at 93.726 117.348) (size 0.8) (drill 0.4) (layers "F.Cu" "B.Cu") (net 1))
 (via (at 102.997 113.03) (size 0.8) (drill 0.4) (layers "F.Cu" "B.Cu") (free) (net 1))
 (via (at 100.076 113.03) (size 0.8) (drill 0.4) (layers "F.Cu" "B.Cu") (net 1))
 (segment (start 98.425 113.157) (end 96.647 114.935) (width 0.5) (layer "B.Cu") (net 1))
 (segment (start 120.142 97.663) (end 108.077 97.663) (width 0.5) (layer "B.Cu") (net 1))
 (segment (start 102.997 113.03) (end 98.552 113.03) (width 0.5) (layer "B.Cu") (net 1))
 (segment (start 107.828 97.414) (end 107.828 95.123) (width 0.5) (layer "B.Cu") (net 1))
 (segment (start 95.631 117.348) (end 93.726 117.348) (width 0.5) (layer "B.Cu") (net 1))
 (segment (start 119.285 87.408) (end 120.396 88.519) (width 0.5) (layer "B.Cu") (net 1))
 (segment (start 120.396 97.409) (end 120.142 97.663) (width 0.5) (layer "B.Cu") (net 1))
 (segment (start 116.84 87.408) (end 119.285 87.408) (width 0.5) (layer "B.Cu") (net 1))
 (segment (start 108.077 97.663) (end 107.828 97.414) (width 0.5) (layer "B.Cu") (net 1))
 (segment (start 96.647 114.935) (end 96.647 116.332) (width 0.5) (layer "B.Cu") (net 1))
 (segment (start 96.647 116.332) (end 95.631 117.348) (width 0.5) (layer "B.Cu") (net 1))
 (segment (start 98.552 113.03) (end 98.425 113.157) (width 0.5) (layer "B.Cu") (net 1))
 (segment (start 120.396 88.519) (end 120.396 97.409) (width 0.5) (layer "B.Cu") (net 1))
 (segment (start 111.76 91.435) (end 111.76 87.408) (width 0.5) (layer "F.Cu") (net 3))
 (segment (start 111.826 91.501) (end 111.76 91.435) (width 0.5) (layer "F.Cu") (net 3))
 (segment (start 115.448 95.123) (end 111.826 91.501) (width 0.5) (layer "F.Cu") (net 3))
 (via (at 111.826 91.501) (size 0.8) (drill 0.4) (layers "F.Cu" "B.Cu") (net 3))
 (segment (start 111.506 91.821) (end 96.751 91.821) (width 0.5) (layer "B.Cu") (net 3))
 (segment (start 96.751 91.821) (end 95.608 92.964) (width 0.5) (layer "B.Cu") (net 3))
 (segment (start 111.826 91.501) (end 111.506 91.821) (width 0.5) (layer "B.Cu") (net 3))
 (segment (start 109.22 91.435) (end 99.677 91.435) (width 0.5) (layer "F.Cu") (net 4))
 (segment (start 112.908 95.123) (end 109.22 91.435) (width 0.5) (layer "F.Cu") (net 4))
 (segment (start 109.22 91.435) (end 109.22 87.408) (width 0.5) (layer "F.Cu") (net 4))
 (segment (start 99.677 91.435) (end 95.608 95.504) (width 0.5) (layer "F.Cu") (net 4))
 (segment (start 95.608 95.504) (end 95.885 95.504) (width 0.5) (layer "F.Cu") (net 4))
 (segment (start 103.235 95.504) (end 104.521 95.504) (width 0.5) (layer "F.Cu") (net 15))
 (via (at 104.521 95.504) (size 0.8) (drill 0.4) (layers "F.Cu" "B.Cu") (free) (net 15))
 (segment (start 100.815 92.837) (end 95.608 98.044) (width 0.5) (layer "B.Cu") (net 15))
 (segment (start 110.368 95.123) (end 108.082 92.837) (width 0.5) (layer "B.Cu") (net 15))
 (segment (start 108.082 92.837) (end 104.775 92.837) (width 0.5) (layer "B.Cu") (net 15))
 (segment (start 104.521 93.091) (end 104.775 92.837) (width 0.5) (layer "B.Cu") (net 15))
 (segment (start 104.775 92.837) (end 100.815 92.837) (width 0.5) (layer "B.Cu") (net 15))
 (segment (start 104.521 95.504) (end 104.521 93.091) (width 0.5) (layer "B.Cu") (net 15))
 (segment (start 103.092 111.157) (end 103.092 107.95) (width 0.5) (layer "F.Cu") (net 20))
 (segment (start 101.031 111.948) (end 101.473 111.506) (width 0.5) (layer "F.Cu") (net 20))
 (segment (start 102.743 111.506) (end 103.092 111.157) (width 0.5) (layer "F.Cu") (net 20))
 (segment (start 101.031 114.6325) (end 101.031 111.948) (width 0.5) (layer "F.Cu") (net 20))
 (segment (start 101.473 111.506) (end 102.743 111.506) (width 0.5) (layer "F.Cu") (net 20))
 (segment (start 103.119 104.748) (end 103.092 104.775) (width 0.5) (layer "F.Cu") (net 25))
 (segment (start 103.119 102.362) (end 103.119 104.748) (width 0.5) (layer "F.Cu") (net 25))
 (segment (start 88.646 119.55) (end 91.1555 119.55) (width 0.5) (layer "F.Cu") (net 22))
 (segment (start 91.1555 119.55) (end 91.3915 119.314) (width 0.5) (layer "F.Cu") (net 22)))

